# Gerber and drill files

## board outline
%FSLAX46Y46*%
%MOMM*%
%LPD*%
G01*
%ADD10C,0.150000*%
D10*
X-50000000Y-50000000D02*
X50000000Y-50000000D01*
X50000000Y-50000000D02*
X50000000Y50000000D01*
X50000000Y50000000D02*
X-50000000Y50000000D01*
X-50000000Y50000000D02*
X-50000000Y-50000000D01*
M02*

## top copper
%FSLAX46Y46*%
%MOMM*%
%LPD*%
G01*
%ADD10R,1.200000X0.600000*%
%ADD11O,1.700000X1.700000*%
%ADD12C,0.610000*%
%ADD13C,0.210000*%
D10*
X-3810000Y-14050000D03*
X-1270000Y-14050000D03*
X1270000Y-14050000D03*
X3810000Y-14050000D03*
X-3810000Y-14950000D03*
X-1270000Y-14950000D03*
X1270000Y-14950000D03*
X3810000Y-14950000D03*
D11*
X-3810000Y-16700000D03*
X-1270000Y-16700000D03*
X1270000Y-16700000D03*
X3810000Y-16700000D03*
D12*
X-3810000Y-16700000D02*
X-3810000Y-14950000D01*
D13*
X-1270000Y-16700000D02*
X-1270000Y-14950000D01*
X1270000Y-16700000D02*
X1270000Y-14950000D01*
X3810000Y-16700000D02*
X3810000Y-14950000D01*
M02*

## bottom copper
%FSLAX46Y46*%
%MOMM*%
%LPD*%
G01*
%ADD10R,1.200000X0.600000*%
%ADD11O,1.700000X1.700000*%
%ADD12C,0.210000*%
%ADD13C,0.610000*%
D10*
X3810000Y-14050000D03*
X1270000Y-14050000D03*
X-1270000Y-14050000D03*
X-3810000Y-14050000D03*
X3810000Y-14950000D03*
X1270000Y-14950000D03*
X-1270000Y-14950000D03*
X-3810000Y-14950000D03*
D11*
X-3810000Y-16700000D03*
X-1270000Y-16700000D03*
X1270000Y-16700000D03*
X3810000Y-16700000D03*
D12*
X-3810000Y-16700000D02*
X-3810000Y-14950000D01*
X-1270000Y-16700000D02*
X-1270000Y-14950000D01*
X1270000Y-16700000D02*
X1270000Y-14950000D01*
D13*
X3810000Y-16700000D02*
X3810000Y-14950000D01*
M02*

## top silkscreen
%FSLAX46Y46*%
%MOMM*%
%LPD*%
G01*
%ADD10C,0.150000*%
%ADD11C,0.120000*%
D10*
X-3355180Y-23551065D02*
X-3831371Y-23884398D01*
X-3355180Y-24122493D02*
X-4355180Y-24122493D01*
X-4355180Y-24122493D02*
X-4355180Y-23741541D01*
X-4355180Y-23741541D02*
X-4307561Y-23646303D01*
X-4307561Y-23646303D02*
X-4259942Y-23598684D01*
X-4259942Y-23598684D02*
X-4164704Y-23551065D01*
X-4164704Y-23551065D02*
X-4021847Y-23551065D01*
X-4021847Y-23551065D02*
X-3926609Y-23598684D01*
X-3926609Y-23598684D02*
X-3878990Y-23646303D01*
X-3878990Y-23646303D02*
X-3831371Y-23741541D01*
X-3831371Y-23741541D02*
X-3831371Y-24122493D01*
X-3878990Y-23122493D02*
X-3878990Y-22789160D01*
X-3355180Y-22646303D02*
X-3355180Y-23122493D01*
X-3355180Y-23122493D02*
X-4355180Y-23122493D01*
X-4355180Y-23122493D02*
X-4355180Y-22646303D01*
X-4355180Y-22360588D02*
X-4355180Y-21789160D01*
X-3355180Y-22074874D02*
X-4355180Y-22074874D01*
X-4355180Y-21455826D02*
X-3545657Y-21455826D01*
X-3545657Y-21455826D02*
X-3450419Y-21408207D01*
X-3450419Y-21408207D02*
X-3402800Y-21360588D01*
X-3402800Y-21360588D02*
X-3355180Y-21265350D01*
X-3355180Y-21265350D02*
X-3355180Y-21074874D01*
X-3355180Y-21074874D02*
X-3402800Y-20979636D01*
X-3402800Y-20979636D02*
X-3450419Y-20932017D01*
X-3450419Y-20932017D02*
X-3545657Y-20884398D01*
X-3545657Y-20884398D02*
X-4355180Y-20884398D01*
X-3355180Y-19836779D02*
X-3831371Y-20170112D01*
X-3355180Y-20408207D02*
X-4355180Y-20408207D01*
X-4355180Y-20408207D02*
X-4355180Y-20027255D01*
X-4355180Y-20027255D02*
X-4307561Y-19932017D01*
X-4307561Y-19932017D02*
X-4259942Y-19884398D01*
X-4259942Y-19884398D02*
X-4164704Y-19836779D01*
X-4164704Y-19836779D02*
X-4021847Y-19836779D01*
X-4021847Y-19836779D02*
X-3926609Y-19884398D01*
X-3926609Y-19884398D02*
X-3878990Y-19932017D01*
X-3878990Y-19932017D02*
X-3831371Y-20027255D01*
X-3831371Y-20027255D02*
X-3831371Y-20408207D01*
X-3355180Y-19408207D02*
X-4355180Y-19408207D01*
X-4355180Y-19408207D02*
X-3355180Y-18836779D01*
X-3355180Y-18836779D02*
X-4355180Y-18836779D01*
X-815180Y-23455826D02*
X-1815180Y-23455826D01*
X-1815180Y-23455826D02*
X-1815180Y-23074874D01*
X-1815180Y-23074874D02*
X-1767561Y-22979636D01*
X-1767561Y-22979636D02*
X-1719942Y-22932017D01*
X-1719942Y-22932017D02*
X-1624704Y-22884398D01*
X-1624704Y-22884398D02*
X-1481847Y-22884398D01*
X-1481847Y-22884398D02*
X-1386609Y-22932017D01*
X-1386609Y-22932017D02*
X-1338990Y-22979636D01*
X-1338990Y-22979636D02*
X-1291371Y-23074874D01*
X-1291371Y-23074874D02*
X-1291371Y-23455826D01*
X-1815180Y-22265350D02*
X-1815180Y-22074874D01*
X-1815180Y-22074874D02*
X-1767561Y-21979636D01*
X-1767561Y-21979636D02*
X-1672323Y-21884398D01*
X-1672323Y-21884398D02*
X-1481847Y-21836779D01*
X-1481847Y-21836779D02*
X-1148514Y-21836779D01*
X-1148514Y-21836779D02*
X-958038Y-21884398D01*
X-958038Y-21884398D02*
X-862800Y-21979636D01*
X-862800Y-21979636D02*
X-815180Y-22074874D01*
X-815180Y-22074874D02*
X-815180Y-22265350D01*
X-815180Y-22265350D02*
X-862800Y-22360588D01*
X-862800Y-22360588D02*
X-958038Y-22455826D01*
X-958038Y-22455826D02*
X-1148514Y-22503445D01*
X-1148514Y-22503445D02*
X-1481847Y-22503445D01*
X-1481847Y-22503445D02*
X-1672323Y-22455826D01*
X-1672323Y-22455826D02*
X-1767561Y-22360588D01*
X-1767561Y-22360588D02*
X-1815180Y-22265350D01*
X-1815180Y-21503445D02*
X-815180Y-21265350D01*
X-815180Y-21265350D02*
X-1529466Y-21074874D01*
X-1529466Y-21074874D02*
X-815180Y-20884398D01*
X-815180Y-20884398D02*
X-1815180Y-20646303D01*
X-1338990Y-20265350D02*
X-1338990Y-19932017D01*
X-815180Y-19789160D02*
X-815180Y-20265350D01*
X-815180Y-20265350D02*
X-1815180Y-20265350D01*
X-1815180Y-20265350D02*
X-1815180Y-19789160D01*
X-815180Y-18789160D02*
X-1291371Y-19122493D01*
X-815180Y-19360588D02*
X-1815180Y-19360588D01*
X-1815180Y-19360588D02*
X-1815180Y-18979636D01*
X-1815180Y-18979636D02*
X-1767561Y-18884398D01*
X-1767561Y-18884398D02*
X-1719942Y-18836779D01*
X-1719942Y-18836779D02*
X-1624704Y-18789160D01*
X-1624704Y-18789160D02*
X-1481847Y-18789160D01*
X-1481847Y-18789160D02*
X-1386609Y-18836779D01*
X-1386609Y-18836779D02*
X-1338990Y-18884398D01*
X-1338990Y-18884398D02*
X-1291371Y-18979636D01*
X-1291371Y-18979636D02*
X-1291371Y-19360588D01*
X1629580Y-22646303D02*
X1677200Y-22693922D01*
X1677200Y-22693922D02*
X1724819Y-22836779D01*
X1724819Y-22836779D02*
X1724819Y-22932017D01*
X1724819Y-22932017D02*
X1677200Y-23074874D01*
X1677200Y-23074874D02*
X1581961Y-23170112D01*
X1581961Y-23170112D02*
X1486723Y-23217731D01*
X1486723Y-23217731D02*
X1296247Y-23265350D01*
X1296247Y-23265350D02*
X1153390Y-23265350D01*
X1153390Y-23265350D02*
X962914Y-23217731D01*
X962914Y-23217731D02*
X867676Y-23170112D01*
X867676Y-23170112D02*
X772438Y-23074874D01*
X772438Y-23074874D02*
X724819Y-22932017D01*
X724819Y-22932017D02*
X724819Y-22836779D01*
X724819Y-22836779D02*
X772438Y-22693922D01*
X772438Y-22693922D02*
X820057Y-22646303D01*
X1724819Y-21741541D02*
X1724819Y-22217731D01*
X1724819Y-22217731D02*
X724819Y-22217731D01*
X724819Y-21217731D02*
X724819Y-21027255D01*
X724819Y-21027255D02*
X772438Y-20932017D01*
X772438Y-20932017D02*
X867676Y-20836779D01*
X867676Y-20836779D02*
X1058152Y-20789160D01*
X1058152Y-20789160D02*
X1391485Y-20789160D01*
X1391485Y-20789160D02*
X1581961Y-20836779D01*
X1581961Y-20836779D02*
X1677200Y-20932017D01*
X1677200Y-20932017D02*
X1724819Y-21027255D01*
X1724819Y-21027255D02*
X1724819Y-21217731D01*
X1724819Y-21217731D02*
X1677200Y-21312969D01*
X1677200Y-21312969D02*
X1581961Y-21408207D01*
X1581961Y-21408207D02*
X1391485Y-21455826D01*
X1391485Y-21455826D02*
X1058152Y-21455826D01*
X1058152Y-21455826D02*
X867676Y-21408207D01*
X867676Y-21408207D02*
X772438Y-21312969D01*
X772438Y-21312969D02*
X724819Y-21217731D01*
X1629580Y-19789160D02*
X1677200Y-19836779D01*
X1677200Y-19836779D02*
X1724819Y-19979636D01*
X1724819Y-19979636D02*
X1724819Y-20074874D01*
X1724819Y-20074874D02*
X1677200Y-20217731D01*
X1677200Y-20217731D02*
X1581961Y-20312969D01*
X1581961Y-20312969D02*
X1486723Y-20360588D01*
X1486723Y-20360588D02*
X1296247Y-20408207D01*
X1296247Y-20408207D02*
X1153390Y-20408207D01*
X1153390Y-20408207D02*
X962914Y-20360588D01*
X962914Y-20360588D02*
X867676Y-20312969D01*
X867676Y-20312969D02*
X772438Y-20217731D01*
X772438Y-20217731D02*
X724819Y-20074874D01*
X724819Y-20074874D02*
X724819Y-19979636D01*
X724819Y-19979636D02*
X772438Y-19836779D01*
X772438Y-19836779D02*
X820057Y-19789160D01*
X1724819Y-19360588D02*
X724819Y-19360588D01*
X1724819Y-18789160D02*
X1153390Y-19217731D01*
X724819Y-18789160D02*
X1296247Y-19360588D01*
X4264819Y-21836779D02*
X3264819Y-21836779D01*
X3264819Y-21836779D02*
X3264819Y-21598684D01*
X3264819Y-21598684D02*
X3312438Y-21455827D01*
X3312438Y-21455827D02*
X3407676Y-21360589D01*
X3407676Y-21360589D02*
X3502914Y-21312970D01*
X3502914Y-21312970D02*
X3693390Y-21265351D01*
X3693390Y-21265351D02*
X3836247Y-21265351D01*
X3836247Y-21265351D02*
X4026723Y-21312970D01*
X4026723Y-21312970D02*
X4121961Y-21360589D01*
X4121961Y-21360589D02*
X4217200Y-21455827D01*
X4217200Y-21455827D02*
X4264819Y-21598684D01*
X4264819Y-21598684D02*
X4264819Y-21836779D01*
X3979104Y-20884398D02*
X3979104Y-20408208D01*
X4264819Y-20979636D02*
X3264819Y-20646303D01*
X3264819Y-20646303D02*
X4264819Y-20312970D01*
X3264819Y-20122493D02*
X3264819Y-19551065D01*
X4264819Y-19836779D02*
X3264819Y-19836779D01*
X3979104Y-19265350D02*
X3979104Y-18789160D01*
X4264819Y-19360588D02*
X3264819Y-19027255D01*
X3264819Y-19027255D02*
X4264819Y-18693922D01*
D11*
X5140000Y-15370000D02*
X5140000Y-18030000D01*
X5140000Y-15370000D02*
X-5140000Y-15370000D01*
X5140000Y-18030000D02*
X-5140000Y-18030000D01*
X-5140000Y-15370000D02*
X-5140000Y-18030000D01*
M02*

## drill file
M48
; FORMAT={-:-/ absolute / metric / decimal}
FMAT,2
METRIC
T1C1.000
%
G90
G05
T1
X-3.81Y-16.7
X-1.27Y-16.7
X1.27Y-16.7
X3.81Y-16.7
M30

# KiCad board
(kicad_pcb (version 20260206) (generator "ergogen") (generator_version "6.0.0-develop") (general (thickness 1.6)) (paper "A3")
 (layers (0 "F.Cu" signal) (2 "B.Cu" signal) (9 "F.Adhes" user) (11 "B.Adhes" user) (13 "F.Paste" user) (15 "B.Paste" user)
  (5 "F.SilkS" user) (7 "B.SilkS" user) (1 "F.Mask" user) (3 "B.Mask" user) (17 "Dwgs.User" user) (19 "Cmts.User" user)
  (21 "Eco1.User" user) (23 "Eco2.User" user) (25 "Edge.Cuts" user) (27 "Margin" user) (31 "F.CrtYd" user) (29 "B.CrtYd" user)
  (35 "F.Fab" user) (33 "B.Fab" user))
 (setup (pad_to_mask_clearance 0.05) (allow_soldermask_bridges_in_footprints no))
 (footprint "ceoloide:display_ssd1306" (layer "B.Cu") (at 0 0 0)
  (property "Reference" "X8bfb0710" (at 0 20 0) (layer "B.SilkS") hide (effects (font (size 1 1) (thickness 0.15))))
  (fp_line (start 5.14 15.37) (end 5.14 18.03) (layer "F.SilkS") (stroke (width 0.12) (type solid)))
  (fp_line (start 5.14 15.37) (end -5.14 15.37) (layer "F.SilkS") (stroke (width 0.12) (type solid)))
  (fp_line (start 5.14 18.03) (end -5.14 18.03) (layer "F.SilkS") (stroke (width 0.12) (type solid)))
  (fp_line (start -5.14 15.37) (end -5.14 18.03) (layer "F.SilkS") (stroke (width 0.12) (type solid)))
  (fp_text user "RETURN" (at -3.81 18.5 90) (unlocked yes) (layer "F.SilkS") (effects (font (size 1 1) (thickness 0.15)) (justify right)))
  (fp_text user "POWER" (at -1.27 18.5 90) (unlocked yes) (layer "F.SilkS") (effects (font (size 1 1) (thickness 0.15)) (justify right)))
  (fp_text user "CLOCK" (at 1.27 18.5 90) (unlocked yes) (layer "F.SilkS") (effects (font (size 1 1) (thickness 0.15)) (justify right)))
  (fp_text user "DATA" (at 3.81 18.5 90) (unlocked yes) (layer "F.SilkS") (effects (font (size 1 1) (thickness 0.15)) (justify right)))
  (pad "14" smd rect (at -3.81 14.05 90) (size 0.6 1.2) (layers "F.Cu" "F.Paste" "F.Mask") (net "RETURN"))
  (pad "15" smd rect (at -1.27 14.05 90) (size 0.6 1.2) (layers "F.Cu" "F.Paste" "F.Mask") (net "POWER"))
  (pad "16" smd rect (at 1.27 14.05 90) (size 0.6 1.2) (layers "F.Cu" "F.Paste" "F.Mask") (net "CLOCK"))
  (pad "17" smd rect (at 3.81 14.05 90) (size 0.6 1.2) (layers "F.Cu" "F.Paste" "F.Mask") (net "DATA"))
  (pad "10" smd rect (at -3.81 14.95 90) (size 0.6 1.2) (layers "F.Cu" "F.Paste" "F.Mask") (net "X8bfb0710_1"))
  (pad "11" smd rect (at -1.27 14.95 90) (size 0.6 1.2) (layers "F.Cu" "F.Paste" "F.Mask") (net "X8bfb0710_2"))
  (pad "12" smd rect (at 1.27 14.95 90) (size 0.6 1.2) (layers "F.Cu" "F.Paste" "F.Mask") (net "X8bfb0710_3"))
  (pad "13" smd rect (at 3.81 14.95 90) (size 0.6 1.2) (layers "F.Cu" "F.Paste" "F.Mask") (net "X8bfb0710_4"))
  (pad "24" smd rect (at 3.81 14.05 270) (size 0.6 1.2) (layers "B.Cu" "B.Paste" "B.Mask") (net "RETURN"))
  (pad "25" smd rect (at 1.27 14.05 270) (size 0.6 1.2) (layers "B.Cu" "B.Paste" "B.Mask") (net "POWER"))
  (pad "26" smd rect (at -1.27 14.05 270) (size 0.6 1.2) (layers "B.Cu" "B.Paste" "B.Mask") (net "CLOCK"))
  (pad "27" smd rect (at -3.81 14.05 270) (size 0.6 1.2) (layers "B.Cu" "B.Paste" "B.Mask") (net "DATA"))
  (pad "20" smd rect (at 3.81 14.95 270) (size 0.6 1.2) (layers "B.Cu" "B.Paste" "B.Mask") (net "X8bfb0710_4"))
  (pad "21" smd rect (at 1.27 14.95 270) (size 0.6 1.2) (layers "B.Cu" "B.Paste" "B.Mask") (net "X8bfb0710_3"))
  (pad "22" smd rect (at -1.27 14.95 270) (size 0.6 1.2) (layers "B.Cu" "B.Paste" "B.Mask") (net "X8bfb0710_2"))
  (pad "23" smd rect (at -3.81 14.95 270) (size 0.6 1.2) (layers "B.Cu" "B.Paste" "B.Mask") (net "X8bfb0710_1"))
  (pad "1" thru_hole oval (at -3.81 16.7 270) (size 1.7 1.7) (drill 1) (layers "*.Cu" "*.Mask") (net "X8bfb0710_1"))
  (pad "2" thru_hole oval (at -1.27 16.7 270) (size 1.7 1.7) (drill 1) (layers "*.Cu" "*.Mask") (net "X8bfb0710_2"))
  (pad "3" thru_hole oval (at 1.27 16.7 270) (size 1.7 1.7) (drill 1) (layers "*.Cu" "*.Mask") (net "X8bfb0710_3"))
  (pad "4" thru_hole oval (at 3.81 16.7 270) (size 1.7 1.7) (drill 1) (layers "*.Cu" "*.Mask") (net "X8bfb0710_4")))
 (segment (start -3.81 16.7) (end -3.81 14.95) (width 0.61) (layer "F.Cu") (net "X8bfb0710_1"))
 (segment (start -1.27 16.7) (end -1.27 14.95) (width 0.21) (layer "F.Cu") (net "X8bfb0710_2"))
 (segment (start 1.27 16.7) (end 1.27 14.95) (width 0.21) (layer "F.Cu") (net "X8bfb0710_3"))
 (segment (start 3.81 16.7) (end 3.81 14.95) (width 0.21) (layer "F.Cu") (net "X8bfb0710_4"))
 (segment (start -3.81 16.7) (end -3.81 14.95) (width 0.21) (layer "B.Cu") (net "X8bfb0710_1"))
 (segment (start -1.27 16.7) (end -1.27 14.95) (width 0.21) (layer "B.Cu") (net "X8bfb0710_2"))
 (segment (start 1.27 16.7) (end 1.27 14.95) (width 0.21) (layer "B.Cu") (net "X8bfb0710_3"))
 (segment (start 3.81 16.7) (end 3.81 14.95) (width 0.61) (layer "B.Cu") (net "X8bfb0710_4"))
 (gr_line (start -50 50) (end 50 50) (layer Edge.Cuts) (stroke (width 0.15) (type default)))
 (gr_line (start 50 50) (end 50 -50) (layer Edge.Cuts) (stroke (width 0.15) (type default)))
 (gr_line (start 50 -50) (end -50 -50) (layer Edge.Cuts) (stroke (width 0.15) (type default)))
 (gr_line (start -50 -50) (end -50 50) (layer Edge.Cuts) (stroke (width 0.15) (type default))))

